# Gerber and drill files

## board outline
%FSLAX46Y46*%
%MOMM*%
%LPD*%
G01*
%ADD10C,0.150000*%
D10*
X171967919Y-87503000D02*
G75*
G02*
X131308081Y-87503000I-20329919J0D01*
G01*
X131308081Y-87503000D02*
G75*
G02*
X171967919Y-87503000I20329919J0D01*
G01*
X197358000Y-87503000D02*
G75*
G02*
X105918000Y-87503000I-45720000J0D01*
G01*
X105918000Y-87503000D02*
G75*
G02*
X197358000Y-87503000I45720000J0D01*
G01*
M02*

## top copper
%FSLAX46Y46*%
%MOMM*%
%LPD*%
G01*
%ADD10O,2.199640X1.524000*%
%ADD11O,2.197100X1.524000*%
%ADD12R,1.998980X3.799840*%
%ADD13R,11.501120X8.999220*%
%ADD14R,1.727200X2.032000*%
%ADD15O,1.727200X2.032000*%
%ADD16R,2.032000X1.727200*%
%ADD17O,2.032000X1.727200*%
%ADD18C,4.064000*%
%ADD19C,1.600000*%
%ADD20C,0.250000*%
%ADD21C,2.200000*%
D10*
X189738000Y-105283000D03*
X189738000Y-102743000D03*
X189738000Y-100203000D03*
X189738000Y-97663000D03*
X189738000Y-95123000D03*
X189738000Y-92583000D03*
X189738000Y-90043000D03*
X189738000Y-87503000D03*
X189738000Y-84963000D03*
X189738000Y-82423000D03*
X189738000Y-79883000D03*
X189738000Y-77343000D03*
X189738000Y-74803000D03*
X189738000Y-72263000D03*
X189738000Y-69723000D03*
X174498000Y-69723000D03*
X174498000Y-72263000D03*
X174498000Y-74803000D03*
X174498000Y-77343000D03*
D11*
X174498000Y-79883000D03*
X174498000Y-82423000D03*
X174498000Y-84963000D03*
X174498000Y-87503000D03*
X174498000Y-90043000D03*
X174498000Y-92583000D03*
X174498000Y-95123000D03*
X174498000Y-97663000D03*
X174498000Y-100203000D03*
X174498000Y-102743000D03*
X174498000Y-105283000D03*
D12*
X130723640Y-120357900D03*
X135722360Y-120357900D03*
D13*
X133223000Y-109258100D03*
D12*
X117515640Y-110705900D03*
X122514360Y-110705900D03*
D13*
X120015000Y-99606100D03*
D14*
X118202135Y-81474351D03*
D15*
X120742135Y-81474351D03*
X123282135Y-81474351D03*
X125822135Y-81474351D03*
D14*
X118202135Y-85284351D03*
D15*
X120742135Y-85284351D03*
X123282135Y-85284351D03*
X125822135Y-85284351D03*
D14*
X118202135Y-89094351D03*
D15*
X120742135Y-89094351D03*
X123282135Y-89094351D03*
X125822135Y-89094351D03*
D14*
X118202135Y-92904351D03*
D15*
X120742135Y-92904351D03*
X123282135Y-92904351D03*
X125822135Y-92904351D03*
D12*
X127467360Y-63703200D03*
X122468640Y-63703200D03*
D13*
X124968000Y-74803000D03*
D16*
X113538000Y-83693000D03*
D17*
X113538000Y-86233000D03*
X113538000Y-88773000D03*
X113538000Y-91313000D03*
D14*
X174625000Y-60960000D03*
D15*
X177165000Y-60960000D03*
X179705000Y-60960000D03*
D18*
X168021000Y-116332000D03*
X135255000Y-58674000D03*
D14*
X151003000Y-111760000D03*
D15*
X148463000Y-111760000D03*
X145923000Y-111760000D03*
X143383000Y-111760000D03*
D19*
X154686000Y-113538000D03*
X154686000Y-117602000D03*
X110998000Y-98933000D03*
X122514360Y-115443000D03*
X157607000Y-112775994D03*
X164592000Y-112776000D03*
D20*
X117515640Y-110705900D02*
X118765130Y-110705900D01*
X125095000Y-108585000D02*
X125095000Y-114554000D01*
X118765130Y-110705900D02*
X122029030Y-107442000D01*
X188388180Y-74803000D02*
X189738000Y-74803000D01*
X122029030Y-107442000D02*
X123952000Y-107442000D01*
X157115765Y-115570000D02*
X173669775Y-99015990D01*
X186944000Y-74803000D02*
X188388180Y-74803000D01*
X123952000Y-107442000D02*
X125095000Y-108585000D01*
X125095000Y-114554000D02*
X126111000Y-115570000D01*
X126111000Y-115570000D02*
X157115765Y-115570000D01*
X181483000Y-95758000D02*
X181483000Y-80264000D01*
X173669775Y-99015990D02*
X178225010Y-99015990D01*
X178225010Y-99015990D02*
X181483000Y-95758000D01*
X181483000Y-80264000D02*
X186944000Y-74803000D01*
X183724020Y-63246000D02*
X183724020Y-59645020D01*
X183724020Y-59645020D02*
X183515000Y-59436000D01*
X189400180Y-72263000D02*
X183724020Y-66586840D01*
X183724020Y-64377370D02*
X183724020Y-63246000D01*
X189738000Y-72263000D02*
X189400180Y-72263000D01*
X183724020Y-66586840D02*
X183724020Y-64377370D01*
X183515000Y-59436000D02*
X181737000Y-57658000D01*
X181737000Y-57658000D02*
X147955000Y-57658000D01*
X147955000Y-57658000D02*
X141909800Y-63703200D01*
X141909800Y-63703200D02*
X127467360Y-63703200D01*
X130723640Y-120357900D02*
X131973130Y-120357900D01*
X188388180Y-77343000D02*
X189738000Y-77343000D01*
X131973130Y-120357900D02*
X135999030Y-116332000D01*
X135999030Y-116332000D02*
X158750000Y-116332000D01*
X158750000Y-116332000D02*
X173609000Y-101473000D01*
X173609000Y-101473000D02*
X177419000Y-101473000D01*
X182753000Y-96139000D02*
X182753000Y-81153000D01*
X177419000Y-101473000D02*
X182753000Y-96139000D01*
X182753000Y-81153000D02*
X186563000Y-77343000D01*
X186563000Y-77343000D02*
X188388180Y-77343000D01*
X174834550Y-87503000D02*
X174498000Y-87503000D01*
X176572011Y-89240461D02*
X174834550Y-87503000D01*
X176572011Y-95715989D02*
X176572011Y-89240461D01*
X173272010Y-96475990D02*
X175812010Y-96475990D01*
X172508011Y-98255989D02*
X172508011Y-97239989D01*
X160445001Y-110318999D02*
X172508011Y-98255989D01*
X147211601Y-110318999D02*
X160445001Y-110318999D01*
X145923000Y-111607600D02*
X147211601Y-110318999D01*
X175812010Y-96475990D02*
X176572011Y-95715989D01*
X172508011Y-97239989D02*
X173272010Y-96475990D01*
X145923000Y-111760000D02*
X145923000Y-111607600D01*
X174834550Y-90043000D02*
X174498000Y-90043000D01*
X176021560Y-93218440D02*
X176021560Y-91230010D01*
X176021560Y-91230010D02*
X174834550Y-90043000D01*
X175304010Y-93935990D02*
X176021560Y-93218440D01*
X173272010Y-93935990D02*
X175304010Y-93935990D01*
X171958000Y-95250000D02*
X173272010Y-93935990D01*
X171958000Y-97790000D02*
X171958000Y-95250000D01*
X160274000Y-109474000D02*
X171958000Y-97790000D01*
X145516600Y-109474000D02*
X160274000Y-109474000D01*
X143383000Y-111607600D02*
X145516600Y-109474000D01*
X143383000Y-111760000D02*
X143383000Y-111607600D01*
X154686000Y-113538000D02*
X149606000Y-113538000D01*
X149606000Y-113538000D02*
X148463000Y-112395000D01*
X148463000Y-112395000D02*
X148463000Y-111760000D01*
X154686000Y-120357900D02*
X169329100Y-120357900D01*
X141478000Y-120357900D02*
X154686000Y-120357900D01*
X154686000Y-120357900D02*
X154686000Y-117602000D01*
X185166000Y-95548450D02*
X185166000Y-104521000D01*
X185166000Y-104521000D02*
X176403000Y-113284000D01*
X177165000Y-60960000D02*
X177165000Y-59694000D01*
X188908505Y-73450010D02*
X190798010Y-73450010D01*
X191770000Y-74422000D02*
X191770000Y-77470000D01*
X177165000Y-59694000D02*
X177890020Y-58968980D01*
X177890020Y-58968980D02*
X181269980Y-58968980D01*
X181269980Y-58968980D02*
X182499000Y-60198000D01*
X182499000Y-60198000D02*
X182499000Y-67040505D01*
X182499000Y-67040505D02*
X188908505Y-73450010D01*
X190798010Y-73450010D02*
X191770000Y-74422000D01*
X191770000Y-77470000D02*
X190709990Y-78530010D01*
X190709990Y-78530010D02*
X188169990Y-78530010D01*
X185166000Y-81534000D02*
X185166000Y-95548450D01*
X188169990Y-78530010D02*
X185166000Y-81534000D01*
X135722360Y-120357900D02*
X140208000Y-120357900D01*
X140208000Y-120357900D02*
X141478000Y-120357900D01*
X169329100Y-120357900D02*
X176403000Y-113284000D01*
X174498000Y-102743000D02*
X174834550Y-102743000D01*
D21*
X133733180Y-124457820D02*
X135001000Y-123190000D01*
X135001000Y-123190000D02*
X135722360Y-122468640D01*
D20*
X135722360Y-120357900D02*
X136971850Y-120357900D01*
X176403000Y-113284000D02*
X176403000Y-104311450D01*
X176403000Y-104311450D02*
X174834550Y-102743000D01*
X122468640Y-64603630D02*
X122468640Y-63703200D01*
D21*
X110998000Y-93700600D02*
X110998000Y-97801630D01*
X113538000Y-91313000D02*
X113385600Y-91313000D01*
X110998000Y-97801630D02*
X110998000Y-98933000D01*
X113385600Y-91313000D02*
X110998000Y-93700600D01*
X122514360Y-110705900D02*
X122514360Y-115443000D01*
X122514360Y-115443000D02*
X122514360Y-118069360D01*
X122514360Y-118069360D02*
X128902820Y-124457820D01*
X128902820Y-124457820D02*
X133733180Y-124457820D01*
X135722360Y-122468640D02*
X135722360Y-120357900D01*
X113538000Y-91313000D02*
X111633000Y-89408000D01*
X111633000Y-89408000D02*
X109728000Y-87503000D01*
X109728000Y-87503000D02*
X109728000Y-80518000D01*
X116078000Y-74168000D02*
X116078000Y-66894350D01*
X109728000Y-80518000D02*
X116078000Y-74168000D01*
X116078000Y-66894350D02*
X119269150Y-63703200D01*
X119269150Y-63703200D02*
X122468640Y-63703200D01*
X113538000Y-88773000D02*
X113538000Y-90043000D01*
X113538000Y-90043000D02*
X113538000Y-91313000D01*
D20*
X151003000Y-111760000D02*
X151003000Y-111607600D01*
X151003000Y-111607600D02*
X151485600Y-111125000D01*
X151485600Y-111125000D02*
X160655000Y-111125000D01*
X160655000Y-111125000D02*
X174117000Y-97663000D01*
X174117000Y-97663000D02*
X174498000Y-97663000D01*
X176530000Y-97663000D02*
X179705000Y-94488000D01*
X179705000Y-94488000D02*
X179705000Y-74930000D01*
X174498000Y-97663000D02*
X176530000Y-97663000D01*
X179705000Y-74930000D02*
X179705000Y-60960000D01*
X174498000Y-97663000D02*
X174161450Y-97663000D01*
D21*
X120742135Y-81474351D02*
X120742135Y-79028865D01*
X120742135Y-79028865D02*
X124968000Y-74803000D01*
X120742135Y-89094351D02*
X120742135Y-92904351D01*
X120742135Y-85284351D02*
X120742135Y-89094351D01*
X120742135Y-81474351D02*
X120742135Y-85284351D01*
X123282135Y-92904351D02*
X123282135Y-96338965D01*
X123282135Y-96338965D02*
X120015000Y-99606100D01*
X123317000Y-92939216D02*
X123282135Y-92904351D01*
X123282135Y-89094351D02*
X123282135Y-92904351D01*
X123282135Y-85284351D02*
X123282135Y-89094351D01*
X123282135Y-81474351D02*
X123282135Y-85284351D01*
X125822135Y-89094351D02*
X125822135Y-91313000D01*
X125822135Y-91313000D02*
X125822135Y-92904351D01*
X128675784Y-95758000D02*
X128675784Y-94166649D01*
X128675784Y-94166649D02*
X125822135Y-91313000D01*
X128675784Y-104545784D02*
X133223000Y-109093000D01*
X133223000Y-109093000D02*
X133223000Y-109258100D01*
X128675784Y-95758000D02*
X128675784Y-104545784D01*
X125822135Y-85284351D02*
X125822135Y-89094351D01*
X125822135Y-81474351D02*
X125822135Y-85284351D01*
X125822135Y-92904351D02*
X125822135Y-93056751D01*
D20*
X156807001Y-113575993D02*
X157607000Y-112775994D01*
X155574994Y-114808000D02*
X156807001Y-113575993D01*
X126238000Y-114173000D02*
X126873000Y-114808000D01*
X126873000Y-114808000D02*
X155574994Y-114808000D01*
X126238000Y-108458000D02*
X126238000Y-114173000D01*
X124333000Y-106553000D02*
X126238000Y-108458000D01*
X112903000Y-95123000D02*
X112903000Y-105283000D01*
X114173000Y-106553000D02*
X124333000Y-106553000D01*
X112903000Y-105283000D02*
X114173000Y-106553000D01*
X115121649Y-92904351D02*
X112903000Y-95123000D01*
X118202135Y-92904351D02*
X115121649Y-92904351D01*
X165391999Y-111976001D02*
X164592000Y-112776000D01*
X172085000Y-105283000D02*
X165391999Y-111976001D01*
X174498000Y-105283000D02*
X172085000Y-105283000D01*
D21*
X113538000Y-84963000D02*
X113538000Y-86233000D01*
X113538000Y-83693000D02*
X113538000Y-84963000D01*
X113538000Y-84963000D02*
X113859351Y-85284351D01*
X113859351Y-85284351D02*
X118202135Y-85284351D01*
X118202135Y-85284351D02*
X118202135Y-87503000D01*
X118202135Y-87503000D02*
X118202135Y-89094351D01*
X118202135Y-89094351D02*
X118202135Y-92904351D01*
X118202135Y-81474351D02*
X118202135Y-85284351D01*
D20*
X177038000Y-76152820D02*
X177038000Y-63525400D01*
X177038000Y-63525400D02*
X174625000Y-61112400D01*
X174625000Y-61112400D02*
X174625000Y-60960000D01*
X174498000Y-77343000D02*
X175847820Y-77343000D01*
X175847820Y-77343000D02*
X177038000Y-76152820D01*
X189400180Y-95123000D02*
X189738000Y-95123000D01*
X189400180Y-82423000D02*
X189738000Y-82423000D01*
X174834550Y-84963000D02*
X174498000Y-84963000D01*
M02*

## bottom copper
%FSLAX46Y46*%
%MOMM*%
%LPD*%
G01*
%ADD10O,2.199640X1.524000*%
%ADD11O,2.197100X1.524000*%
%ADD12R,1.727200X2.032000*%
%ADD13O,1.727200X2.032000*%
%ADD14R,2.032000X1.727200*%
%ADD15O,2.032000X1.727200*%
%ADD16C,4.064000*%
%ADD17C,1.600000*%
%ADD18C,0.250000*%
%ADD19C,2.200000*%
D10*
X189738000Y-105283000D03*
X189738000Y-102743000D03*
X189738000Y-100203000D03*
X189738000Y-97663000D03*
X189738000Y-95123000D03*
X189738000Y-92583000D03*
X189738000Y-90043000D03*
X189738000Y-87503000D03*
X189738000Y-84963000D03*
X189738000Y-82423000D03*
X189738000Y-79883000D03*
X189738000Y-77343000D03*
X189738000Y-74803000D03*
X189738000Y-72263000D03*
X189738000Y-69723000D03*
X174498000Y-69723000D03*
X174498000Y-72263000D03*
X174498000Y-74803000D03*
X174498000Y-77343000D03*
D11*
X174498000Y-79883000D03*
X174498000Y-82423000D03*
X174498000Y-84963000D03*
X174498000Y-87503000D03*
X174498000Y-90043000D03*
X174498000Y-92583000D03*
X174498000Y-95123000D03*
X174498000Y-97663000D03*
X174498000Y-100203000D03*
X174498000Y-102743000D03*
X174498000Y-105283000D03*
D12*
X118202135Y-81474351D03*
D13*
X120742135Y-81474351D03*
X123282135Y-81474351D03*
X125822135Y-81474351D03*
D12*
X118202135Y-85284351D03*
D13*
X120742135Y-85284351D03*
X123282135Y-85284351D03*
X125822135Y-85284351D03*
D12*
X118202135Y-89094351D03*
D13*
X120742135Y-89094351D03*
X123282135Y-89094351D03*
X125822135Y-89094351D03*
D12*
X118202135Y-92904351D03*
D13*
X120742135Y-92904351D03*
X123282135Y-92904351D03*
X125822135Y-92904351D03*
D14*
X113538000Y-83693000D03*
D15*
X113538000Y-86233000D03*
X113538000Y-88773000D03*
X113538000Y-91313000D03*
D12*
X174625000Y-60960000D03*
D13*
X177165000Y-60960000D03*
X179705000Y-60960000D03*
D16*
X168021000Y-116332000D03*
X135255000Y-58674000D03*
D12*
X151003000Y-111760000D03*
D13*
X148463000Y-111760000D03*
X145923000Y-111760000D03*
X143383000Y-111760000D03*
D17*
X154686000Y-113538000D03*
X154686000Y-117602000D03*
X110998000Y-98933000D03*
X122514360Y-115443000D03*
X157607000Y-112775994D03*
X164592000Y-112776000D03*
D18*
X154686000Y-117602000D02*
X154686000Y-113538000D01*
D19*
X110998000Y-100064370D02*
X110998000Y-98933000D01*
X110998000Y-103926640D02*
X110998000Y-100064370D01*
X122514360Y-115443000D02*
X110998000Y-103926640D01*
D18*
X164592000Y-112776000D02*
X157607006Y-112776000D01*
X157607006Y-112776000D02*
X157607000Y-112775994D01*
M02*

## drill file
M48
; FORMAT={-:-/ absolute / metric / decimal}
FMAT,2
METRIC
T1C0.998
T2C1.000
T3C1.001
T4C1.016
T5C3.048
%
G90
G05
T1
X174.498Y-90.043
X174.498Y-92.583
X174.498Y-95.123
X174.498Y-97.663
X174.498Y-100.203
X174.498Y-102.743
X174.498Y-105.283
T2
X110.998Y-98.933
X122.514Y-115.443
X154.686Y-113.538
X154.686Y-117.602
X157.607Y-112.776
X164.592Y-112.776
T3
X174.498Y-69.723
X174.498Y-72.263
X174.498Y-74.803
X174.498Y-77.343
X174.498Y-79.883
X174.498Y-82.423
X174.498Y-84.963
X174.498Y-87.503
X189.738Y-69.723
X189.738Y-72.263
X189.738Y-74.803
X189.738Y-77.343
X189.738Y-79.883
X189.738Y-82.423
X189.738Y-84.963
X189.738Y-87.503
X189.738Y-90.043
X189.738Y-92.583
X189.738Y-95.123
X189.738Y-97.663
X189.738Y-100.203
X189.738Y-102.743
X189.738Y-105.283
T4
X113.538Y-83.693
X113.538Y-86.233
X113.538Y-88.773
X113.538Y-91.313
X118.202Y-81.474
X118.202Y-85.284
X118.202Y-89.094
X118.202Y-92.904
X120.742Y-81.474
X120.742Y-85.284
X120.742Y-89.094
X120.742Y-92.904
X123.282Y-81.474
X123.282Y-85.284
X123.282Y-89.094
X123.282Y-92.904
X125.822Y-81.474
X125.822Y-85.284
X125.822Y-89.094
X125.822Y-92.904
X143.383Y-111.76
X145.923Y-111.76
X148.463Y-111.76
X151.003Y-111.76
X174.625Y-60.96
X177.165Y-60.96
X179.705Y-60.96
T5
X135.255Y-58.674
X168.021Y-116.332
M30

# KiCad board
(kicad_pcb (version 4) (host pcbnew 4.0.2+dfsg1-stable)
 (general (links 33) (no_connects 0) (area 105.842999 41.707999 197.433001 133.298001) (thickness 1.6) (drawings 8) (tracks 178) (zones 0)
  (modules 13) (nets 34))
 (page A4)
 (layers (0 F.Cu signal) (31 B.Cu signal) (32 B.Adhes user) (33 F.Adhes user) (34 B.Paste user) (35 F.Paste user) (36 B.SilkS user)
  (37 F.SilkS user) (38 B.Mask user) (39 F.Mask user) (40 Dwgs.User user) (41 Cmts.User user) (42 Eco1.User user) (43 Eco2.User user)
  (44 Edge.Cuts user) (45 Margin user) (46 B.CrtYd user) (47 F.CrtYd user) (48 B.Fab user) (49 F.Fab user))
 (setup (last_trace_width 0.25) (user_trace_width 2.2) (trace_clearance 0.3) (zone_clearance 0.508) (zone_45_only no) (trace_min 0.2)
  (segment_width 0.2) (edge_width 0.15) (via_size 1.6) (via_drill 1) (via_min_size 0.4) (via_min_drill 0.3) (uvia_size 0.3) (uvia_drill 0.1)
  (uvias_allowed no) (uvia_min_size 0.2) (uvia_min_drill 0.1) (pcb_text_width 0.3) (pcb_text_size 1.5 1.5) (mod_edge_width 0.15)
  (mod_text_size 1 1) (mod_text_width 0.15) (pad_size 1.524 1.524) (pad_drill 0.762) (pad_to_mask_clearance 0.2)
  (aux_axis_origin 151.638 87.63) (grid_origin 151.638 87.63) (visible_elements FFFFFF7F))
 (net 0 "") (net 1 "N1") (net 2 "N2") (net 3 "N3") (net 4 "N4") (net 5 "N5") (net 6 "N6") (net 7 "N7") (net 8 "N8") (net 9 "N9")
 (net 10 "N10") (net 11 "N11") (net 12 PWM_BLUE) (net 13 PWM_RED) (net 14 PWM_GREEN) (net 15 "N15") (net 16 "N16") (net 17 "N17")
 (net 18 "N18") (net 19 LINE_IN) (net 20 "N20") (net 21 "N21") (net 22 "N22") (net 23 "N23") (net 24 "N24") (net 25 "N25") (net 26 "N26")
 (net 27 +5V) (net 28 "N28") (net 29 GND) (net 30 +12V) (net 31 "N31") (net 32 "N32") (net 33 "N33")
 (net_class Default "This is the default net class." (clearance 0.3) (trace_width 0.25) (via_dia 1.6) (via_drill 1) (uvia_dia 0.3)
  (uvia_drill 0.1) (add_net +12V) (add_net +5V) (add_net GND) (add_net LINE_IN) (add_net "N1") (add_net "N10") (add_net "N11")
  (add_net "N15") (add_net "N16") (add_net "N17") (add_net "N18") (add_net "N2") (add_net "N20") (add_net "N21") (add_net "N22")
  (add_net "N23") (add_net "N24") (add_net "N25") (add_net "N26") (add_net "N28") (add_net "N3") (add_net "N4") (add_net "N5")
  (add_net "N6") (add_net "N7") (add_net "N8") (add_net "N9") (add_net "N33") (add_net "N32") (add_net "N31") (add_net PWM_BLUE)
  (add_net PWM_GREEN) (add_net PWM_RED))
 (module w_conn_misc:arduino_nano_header (layer F.Cu) (at 182.118 87.503 90)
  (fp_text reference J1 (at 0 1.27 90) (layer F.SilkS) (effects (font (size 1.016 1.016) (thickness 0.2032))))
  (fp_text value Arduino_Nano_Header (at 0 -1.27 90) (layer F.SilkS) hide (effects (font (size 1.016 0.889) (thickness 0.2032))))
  (pad 1 thru_hole oval (at -17.78 7.62 90) (size 1.524 2.19964) (drill 1.00076) (layers *.Cu *.Mask F.SilkS) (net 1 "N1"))
  (pad 2 thru_hole oval (at -15.24 7.62 90) (size 1.524 2.19964) (drill 1.00076) (layers *.Cu *.Mask F.SilkS) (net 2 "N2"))
  (pad 3 thru_hole oval (at -12.7 7.62 90) (size 1.524 2.19964) (drill 1.00076) (layers *.Cu *.Mask F.SilkS) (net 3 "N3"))
  (pad 4 thru_hole oval (at -10.16 7.62 90) (size 1.524 2.19964) (drill 1.00076) (layers *.Cu *.Mask F.SilkS) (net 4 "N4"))
  (pad 5 thru_hole oval (at -7.62 7.62 90) (size 1.524 2.19964) (drill 1.00076) (layers *.Cu *.Mask F.SilkS) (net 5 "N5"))
  (pad 6 thru_hole oval (at -5.08 7.62 90) (size 1.524 2.19964) (drill 1.00076) (layers *.Cu *.Mask F.SilkS) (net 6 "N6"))
  (pad 7 thru_hole oval (at -2.54 7.62 90) (size 1.524 2.19964) (drill 1.00076) (layers *.Cu *.Mask F.SilkS) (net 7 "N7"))
  (pad 8 thru_hole oval (at 0 7.62 90) (size 1.524 2.19964) (drill 1.00076) (layers *.Cu *.Mask F.SilkS) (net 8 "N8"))
  (pad 9 thru_hole oval (at 2.54 7.62 90) (size 1.524 2.19964) (drill 1.00076) (layers *.Cu *.Mask F.SilkS) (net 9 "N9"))
  (pad 10 thru_hole oval (at 5.08 7.62 90) (size 1.524 2.19964) (drill 1.00076) (layers *.Cu *.Mask F.SilkS) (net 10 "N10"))
  (pad 11 thru_hole oval (at 7.62 7.62 90) (size 1.524 2.19964) (drill 1.00076) (layers *.Cu *.Mask F.SilkS) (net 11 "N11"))
  (pad 12 thru_hole oval (at 10.16 7.62 90) (size 1.524 2.19964) (drill 1.00076) (layers *.Cu *.Mask F.SilkS) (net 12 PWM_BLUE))
  (pad 13 thru_hole oval (at 12.7 7.62 90) (size 1.524 2.19964) (drill 1.00076) (layers *.Cu *.Mask F.SilkS) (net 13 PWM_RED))
  (pad 14 thru_hole oval (at 15.24 7.62 90) (size 1.524 2.19964) (drill 1.00076) (layers *.Cu *.Mask F.SilkS) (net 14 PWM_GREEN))
  (pad 15 thru_hole oval (at 17.78 7.62 90) (size 1.524 2.19964) (drill 1.00076) (layers *.Cu *.Mask F.SilkS) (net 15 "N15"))
  (pad 16 thru_hole oval (at 17.78 -7.62 90) (size 1.524 2.19964) (drill 1.00076) (layers *.Cu *.Mask F.SilkS) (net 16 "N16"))
  (pad 17 thru_hole oval (at 15.24 -7.62 90) (size 1.524 2.19964) (drill 1.00076) (layers *.Cu *.Mask F.SilkS) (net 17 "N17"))
  (pad 18 thru_hole oval (at 12.7 -7.62 90) (size 1.524 2.19964) (drill 1.00076) (layers *.Cu *.Mask F.SilkS) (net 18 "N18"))
  (pad 19 thru_hole oval (at 10.16 -7.62 90) (size 1.524 2.19964) (drill 1.00076) (layers *.Cu *.Mask F.SilkS) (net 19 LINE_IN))
  (pad 20 thru_hole oval (at 7.62 -7.62 90) (size 1.524 2.1971) (drill 1.00076) (layers *.Cu *.Mask F.SilkS) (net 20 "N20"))
  (pad 21 thru_hole oval (at 5.08 -7.62 90) (size 1.524 2.1971) (drill 1.00076) (layers *.Cu *.Mask F.SilkS) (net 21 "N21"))
  (pad 22 thru_hole oval (at 2.54 -7.62 90) (size 1.524 2.1971) (drill 1.00076) (layers *.Cu *.Mask F.SilkS) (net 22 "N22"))
  (pad 23 thru_hole oval (at 0 -7.62 90) (size 1.524 2.1971) (drill 1.00076) (layers *.Cu *.Mask F.SilkS) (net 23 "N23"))
  (pad 24 thru_hole oval (at -2.54 -7.62 90) (size 1.524 2.1971) (drill 0.99822) (layers *.Cu *.Mask F.SilkS) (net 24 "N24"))
  (pad 25 thru_hole oval (at -5.08 -7.62 90) (size 1.524 2.1971) (drill 0.99822) (layers *.Cu *.Mask F.SilkS) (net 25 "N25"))
  (pad 26 thru_hole oval (at -7.62 -7.62 90) (size 1.524 2.1971) (drill 0.99822) (layers *.Cu *.Mask F.SilkS) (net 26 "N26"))
  (pad 27 thru_hole oval (at -10.16 -7.62 90) (size 1.524 2.1971) (drill 0.99822) (layers *.Cu *.Mask F.SilkS) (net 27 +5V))
  (pad 28 thru_hole oval (at -12.7 -7.62 90) (size 1.524 2.1971) (drill 0.99822) (layers *.Cu *.Mask F.SilkS) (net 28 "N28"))
  (pad 29 thru_hole oval (at -15.24 -7.62 90) (size 1.524 2.1971) (drill 0.99822) (layers *.Cu *.Mask F.SilkS) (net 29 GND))
  (pad 30 thru_hole oval (at -17.78 -7.62 90) (size 1.524 2.1971) (drill 0.99822) (layers *.Cu *.Mask F.SilkS) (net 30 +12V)))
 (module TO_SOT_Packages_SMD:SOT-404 (layer F.Cu) (at 133.223 114.808)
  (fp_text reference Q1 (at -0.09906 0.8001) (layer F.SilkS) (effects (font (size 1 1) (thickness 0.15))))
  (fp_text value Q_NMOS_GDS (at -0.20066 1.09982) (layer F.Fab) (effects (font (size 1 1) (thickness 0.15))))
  (pad 1 smd rect (at -2.49936 5.5499) (size 1.99898 3.79984) (layers F.Cu F.Paste F.Mask) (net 12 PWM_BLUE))
  (pad 3 smd rect (at 2.49936 5.5499) (size 1.99898 3.79984) (layers F.Cu F.Paste F.Mask) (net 29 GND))
  (pad 2 smd rect (at 0 -5.5499) (size 11.50112 8.99922) (layers F.Cu F.Paste F.Mask) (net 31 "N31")))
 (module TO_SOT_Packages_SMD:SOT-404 (layer F.Cu) (at 120.015 105.156)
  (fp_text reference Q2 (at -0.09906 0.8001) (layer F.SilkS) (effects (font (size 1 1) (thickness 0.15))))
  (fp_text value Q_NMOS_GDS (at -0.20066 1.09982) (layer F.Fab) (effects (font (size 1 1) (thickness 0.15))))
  (pad 1 smd rect (at -2.49936 5.5499) (size 1.99898 3.79984) (layers F.Cu F.Paste F.Mask) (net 13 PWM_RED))
  (pad 3 smd rect (at 2.49936 5.5499) (size 1.99898 3.79984) (layers F.Cu F.Paste F.Mask) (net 29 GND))
  (pad 2 smd rect (at 0 -5.5499) (size 11.50112 8.99922) (layers F.Cu F.Paste F.Mask) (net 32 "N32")))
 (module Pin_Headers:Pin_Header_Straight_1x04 (layer F.Cu) (at 118.202135 81.474351 90)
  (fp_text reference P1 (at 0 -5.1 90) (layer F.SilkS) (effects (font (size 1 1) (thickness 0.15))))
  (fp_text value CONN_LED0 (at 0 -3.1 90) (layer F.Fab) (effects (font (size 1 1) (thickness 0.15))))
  (pad 1 thru_hole rect (at 0 0 90) (size 2.032 1.7272) (drill 1.016) (layers *.Cu *.Mask F.SilkS) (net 30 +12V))
  (pad 2 thru_hole oval (at 0 2.54 90) (size 2.032 1.7272) (drill 1.016) (layers *.Cu *.Mask F.SilkS) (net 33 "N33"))
  (pad 3 thru_hole oval (at 0 5.08 90) (size 2.032 1.7272) (drill 1.016) (layers *.Cu *.Mask F.SilkS) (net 32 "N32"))
  (pad 4 thru_hole oval (at 0 7.62 90) (size 2.032 1.7272) (drill 1.016) (layers *.Cu *.Mask F.SilkS) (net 31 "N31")))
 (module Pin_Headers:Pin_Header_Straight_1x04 (layer F.Cu) (at 118.202135 85.284351 90)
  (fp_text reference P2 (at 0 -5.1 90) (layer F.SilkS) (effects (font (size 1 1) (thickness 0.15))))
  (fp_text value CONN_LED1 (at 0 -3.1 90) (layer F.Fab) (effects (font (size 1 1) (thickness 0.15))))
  (pad 1 thru_hole rect (at 0 0 90) (size 2.032 1.7272) (drill 1.016) (layers *.Cu *.Mask F.SilkS) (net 30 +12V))
  (pad 2 thru_hole oval (at 0 2.54 90) (size 2.032 1.7272) (drill 1.016) (layers *.Cu *.Mask F.SilkS) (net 33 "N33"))
  (pad 3 thru_hole oval (at 0 5.08 90) (size 2.032 1.7272) (drill 1.016) (layers *.Cu *.Mask F.SilkS) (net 32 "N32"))
  (pad 4 thru_hole oval (at 0 7.62 90) (size 2.032 1.7272) (drill 1.016) (layers *.Cu *.Mask F.SilkS) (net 31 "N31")))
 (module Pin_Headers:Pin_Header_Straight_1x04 (layer F.Cu) (at 118.202135 89.094351 90)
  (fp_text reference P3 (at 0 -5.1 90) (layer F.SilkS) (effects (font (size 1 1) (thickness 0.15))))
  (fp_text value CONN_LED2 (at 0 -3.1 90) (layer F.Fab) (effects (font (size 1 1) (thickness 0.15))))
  (pad 1 thru_hole rect (at 0 0 90) (size 2.032 1.7272) (drill 1.016) (layers *.Cu *.Mask F.SilkS) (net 30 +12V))
  (pad 2 thru_hole oval (at 0 2.54 90) (size 2.032 1.7272) (drill 1.016) (layers *.Cu *.Mask F.SilkS) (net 33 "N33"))
  (pad 3 thru_hole oval (at 0 5.08 90) (size 2.032 1.7272) (drill 1.016) (layers *.Cu *.Mask F.SilkS) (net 32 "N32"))
  (pad 4 thru_hole oval (at 0 7.62 90) (size 2.032 1.7272) (drill 1.016) (layers *.Cu *.Mask F.SilkS) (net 31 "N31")))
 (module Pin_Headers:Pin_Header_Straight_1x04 (layer F.Cu) (at 118.202135 92.904351 90)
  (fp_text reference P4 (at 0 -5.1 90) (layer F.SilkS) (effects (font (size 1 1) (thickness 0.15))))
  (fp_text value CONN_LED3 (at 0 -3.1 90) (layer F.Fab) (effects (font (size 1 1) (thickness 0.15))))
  (pad 1 thru_hole rect (at 0 0 90) (size 2.032 1.7272) (drill 1.016) (layers *.Cu *.Mask F.SilkS) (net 30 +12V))
  (pad 2 thru_hole oval (at 0 2.54 90) (size 2.032 1.7272) (drill 1.016) (layers *.Cu *.Mask F.SilkS) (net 33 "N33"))
  (pad 3 thru_hole oval (at 0 5.08 90) (size 2.032 1.7272) (drill 1.016) (layers *.Cu *.Mask F.SilkS) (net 32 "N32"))
  (pad 4 thru_hole oval (at 0 7.62 90) (size 2.032 1.7272) (drill 1.016) (layers *.Cu *.Mask F.SilkS) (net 31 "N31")))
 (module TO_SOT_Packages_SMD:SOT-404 (layer F.Cu) (at 124.968 69.2531 180)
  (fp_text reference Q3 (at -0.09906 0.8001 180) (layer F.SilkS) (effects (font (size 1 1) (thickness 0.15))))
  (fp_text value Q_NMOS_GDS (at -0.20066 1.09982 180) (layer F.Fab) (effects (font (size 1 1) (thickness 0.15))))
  (pad 1 smd rect (at -2.49936 5.5499 180) (size 1.99898 3.79984) (layers F.Cu F.Paste F.Mask) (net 14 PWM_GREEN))
  (pad 3 smd rect (at 2.49936 5.5499 180) (size 1.99898 3.79984) (layers F.Cu F.Paste F.Mask) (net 29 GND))
  (pad 2 smd rect (at 0 -5.5499 180) (size 11.50112 8.99922) (layers F.Cu F.Paste F.Mask) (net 33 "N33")))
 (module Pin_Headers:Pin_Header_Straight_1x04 (layer F.Cu) (at 113.538 83.693)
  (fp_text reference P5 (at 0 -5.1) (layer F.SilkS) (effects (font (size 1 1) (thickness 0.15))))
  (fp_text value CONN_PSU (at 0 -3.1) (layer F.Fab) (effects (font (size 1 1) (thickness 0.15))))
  (pad 1 thru_hole rect (at 0 0) (size 2.032 1.7272) (drill 1.016) (layers *.Cu *.Mask F.SilkS) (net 30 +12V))
  (pad 2 thru_hole oval (at 0 2.54) (size 2.032 1.7272) (drill 1.016) (layers *.Cu *.Mask F.SilkS) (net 30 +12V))
  (pad 3 thru_hole oval (at 0 5.08) (size 2.032 1.7272) (drill 1.016) (layers *.Cu *.Mask F.SilkS) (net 29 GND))
  (pad 4 thru_hole oval (at 0 7.62) (size 2.032 1.7272) (drill 1.016) (layers *.Cu *.Mask F.SilkS) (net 29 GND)))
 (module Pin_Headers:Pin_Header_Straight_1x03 (layer F.Cu) (at 174.625 60.96 90)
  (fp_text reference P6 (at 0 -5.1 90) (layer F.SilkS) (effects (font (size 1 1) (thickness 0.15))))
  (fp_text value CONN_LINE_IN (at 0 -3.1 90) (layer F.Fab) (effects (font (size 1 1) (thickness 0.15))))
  (pad 1 thru_hole rect (at 0 0 90) (size 2.032 1.7272) (drill 1.016) (layers *.Cu *.Mask F.SilkS) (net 19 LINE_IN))
  (pad 2 thru_hole oval (at 0 2.54 90) (size 2.032 1.7272) (drill 1.016) (layers *.Cu *.Mask F.SilkS) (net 29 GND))
  (pad 3 thru_hole oval (at 0 5.08 90) (size 2.032 1.7272) (drill 1.016) (layers *.Cu *.Mask F.SilkS) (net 27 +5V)))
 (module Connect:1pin (layer F.Cu) (at 168.021 116.332)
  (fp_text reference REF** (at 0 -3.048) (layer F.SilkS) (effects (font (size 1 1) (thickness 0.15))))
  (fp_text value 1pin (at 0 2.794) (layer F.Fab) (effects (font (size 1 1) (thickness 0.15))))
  (pad 1 thru_hole circle (at 0 0) (size 4.064 4.064) (drill 3.048) (layers *.Cu *.Mask F.SilkS)))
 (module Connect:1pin (layer F.Cu) (at 135.255 58.674)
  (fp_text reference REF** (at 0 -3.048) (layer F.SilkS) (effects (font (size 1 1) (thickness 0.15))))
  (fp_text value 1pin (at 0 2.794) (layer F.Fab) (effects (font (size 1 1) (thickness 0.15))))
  (pad 1 thru_hole circle (at 0 0) (size 4.064 4.064) (drill 3.048) (layers *.Cu *.Mask F.SilkS)))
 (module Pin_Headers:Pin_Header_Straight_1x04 (layer F.Cu) (at 151.003 111.76 270)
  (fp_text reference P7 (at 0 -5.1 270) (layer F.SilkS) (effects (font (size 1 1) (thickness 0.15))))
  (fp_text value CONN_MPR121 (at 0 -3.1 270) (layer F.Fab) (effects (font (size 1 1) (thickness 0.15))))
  (pad 1 thru_hole rect (at 0 0 270) (size 2.032 1.7272) (drill 1.016) (layers *.Cu *.Mask F.SilkS) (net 27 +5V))
  (pad 2 thru_hole oval (at 0 2.54 270) (size 2.032 1.7272) (drill 1.016) (layers *.Cu *.Mask F.SilkS) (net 29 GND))
  (pad 3 thru_hole oval (at 0 5.08 270) (size 2.032 1.7272) (drill 1.016) (layers *.Cu *.Mask F.SilkS) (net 23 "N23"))
  (pad 4 thru_hole oval (at 0 7.62 270) (size 2.032 1.7272) (drill 1.016) (layers *.Cu *.Mask F.SilkS) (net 24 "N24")))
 (gr_circle (center 151.638 87.503) (end 171.958 88.138) (layer Edge.Cuts) (width 0.15))
 (gr_circle (center 151.638 87.503) (end 197.358 87.503) (layer Edge.Cuts) (width 0.15))
 (segment (start 117.51564 110.7059) (end 118.76513 110.7059) (width 0.25) (layer F.Cu) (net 13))
 (segment (start 125.095 108.585) (end 125.095 114.554) (width 0.25) (layer F.Cu) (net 13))
 (segment (start 118.76513 110.7059) (end 122.02903 107.442) (width 0.25) (layer F.Cu) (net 13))
 (segment (start 188.38818 74.803) (end 189.738 74.803) (width 0.25) (layer F.Cu) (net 13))
 (segment (start 122.02903 107.442) (end 123.952 107.442) (width 0.25) (layer F.Cu) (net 13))
 (segment (start 157.115765 115.57) (end 173.669775 99.01599) (width 0.25) (layer F.Cu) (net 13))
 (segment (start 186.944 74.803) (end 188.38818 74.803) (width 0.25) (layer F.Cu) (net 13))
 (segment (start 123.952 107.442) (end 125.095 108.585) (width 0.25) (layer F.Cu) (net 13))
 (segment (start 125.095 114.554) (end 126.111 115.57) (width 0.25) (layer F.Cu) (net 13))
 (segment (start 126.111 115.57) (end 157.115765 115.57) (width 0.25) (layer F.Cu) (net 13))
 (segment (start 181.483 95.758) (end 181.483 80.264) (width 0.25) (layer F.Cu) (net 13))
 (segment (start 173.669775 99.01599) (end 178.22501 99.01599) (width 0.25) (layer F.Cu) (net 13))
 (segment (start 178.22501 99.01599) (end 181.483 95.758) (width 0.25) (layer F.Cu) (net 13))
 (segment (start 181.483 80.264) (end 186.944 74.803) (width 0.25) (layer F.Cu) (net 13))
 (segment (start 183.72402 63.246) (end 183.72402 59.64502) (width 0.25) (layer F.Cu) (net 14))
 (segment (start 183.72402 59.64502) (end 183.515 59.436) (width 0.25) (layer F.Cu) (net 14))
 (segment (start 189.40018 72.263) (end 183.72402 66.58684) (width 0.25) (layer F.Cu) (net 14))
 (segment (start 183.72402 64.37737) (end 183.72402 63.246) (width 0.25) (layer F.Cu) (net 14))
 (segment (start 189.738 72.263) (end 189.40018 72.263) (width 0.25) (layer F.Cu) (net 14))
 (segment (start 183.72402 66.58684) (end 183.72402 64.37737) (width 0.25) (layer F.Cu) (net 14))
 (segment (start 183.515 59.436) (end 181.737 57.658) (width 0.25) (layer F.Cu) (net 14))
 (segment (start 181.737 57.658) (end 147.955 57.658) (width 0.25) (layer F.Cu) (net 14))
 (segment (start 147.955 57.658) (end 141.9098 63.7032) (width 0.25) (layer F.Cu) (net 14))
 (segment (start 141.9098 63.7032) (end 127.46736 63.7032) (width 0.25) (layer F.Cu) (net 14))
 (segment (start 130.72364 120.3579) (end 131.97313 120.3579) (width 0.25) (layer F.Cu) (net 12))
 (segment (start 188.38818 77.343) (end 189.738 77.343) (width 0.25) (layer F.Cu) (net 12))
 (segment (start 131.97313 120.3579) (end 135.99903 116.332) (width 0.25) (layer F.Cu) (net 12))
 (segment (start 135.99903 116.332) (end 158.75 116.332) (width 0.25) (layer F.Cu) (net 12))
 (segment (start 158.75 116.332) (end 173.609 101.473) (width 0.25) (layer F.Cu) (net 12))
 (segment (start 173.609 101.473) (end 177.419 101.473) (width 0.25) (layer F.Cu) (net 12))
 (segment (start 182.753 96.139) (end 182.753 81.153) (width 0.25) (layer F.Cu) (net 12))
 (segment (start 177.419 101.473) (end 182.753 96.139) (width 0.25) (layer F.Cu) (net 12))
 (segment (start 182.753 81.153) (end 186.563 77.343) (width 0.25) (layer F.Cu) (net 12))
 (segment (start 186.563 77.343) (end 188.38818 77.343) (width 0.25) (layer F.Cu) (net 12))
 (segment (start 174.83455 87.503) (end 174.498 87.503) (width 0.25) (layer F.Cu) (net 23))
 (segment (start 176.572011 89.240461) (end 174.83455 87.503) (width 0.25) (layer F.Cu) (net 23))
 (segment (start 176.572011 95.715989) (end 176.572011 89.240461) (width 0.25) (layer F.Cu) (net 23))
 (segment (start 173.27201 96.47599) (end 175.81201 96.47599) (width 0.25) (layer F.Cu) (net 23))
 (segment (start 172.508011 98.255989) (end 172.508011 97.239989) (width 0.25) (layer F.Cu) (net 23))
 (segment (start 160.445001 110.318999) (end 172.508011 98.255989) (width 0.25) (layer F.Cu) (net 23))
 (segment (start 147.211601 110.318999) (end 160.445001 110.318999) (width 0.25) (layer F.Cu) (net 23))
 (segment (start 145.923 111.6076) (end 147.211601 110.318999) (width 0.25) (layer F.Cu) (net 23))
 (segment (start 175.81201 96.47599) (end 176.572011 95.715989) (width 0.25) (layer F.Cu) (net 23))
 (segment (start 172.508011 97.239989) (end 173.27201 96.47599) (width 0.25) (layer F.Cu) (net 23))
 (segment (start 145.923 111.76) (end 145.923 111.6076) (width 0.25) (layer F.Cu) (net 23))
 (segment (start 174.83455 90.043) (end 174.498 90.043) (width 0.25) (layer F.Cu) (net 24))
 (segment (start 176.02156 93.21844) (end 176.02156 91.23001) (width 0.25) (layer F.Cu) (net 24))
 (segment (start 176.02156 91.23001) (end 174.83455 90.043) (width 0.25) (layer F.Cu) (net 24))
 (segment (start 175.30401 93.93599) (end 176.02156 93.21844) (width 0.25) (layer F.Cu) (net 24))
 (segment (start 173.27201 93.93599) (end 175.30401 93.93599) (width 0.25) (layer F.Cu) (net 24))
 (segment (start 171.958 95.25) (end 173.27201 93.93599) (width 0.25) (layer F.Cu) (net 24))
 (segment (start 171.958 97.79) (end 171.958 95.25) (width 0.25) (layer F.Cu) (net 24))
 (segment (start 160.274 109.474) (end 171.958 97.79) (width 0.25) (layer F.Cu) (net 24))
 (segment (start 145.5166 109.474) (end 160.274 109.474) (width 0.25) (layer F.Cu) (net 24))
 (segment (start 143.383 111.6076) (end 145.5166 109.474) (width 0.25) (layer F.Cu) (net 24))
 (segment (start 143.383 111.76) (end 143.383 111.6076) (width 0.25) (layer F.Cu) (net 24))
 (segment (start 154.686 113.538) (end 149.606 113.538) (width 0.25) (layer F.Cu) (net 29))
 (segment (start 149.606 113.538) (end 148.463 112.395) (width 0.25) (layer F.Cu) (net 29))
 (segment (start 148.463 112.395) (end 148.463 111.76) (width 0.25) (layer F.Cu) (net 29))
 (segment (start 154.686 117.602) (end 154.686 113.538) (width 0.25) (layer B.Cu) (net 29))
 (via (at 154.686 113.538) (size 1.6) (drill 1) (layers F.Cu B.Cu) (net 29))
 (segment (start 154.686 120.3579) (end 169.3291 120.3579) (width 0.25) (layer F.Cu) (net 29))
 (segment (start 141.478 120.3579) (end 154.686 120.3579) (width 0.25) (layer F.Cu) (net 29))
 (segment (start 154.686 120.3579) (end 154.686 117.602) (width 0.25) (layer F.Cu) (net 29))
 (via (at 154.686 117.602) (size 1.6) (drill 1) (layers F.Cu B.Cu) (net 29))
 (segment (start 185.166 95.54845) (end 185.166 104.521) (width 0.25) (layer F.Cu) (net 29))
 (segment (start 185.166 104.521) (end 176.403 113.284) (width 0.25) (layer F.Cu) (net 29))
 (segment (start 177.165 60.96) (end 177.165 59.694) (width 0.25) (layer F.Cu) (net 29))
 (segment (start 188.908505 73.45001) (end 190.79801 73.45001) (width 0.25) (layer F.Cu) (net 29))
 (segment (start 191.77 74.422) (end 191.77 77.47) (width 0.25) (layer F.Cu) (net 29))
 (segment (start 177.165 59.694) (end 177.89002 58.96898) (width 0.25) (layer F.Cu) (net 29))
 (segment (start 177.89002 58.96898) (end 181.26998 58.96898) (width 0.25) (layer F.Cu) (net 29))
 (segment (start 181.26998 58.96898) (end 182.499 60.198) (width 0.25) (layer F.Cu) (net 29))
 (segment (start 182.499 60.198) (end 182.499 67.040505) (width 0.25) (layer F.Cu) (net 29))
 (segment (start 182.499 67.040505) (end 188.908505 73.45001) (width 0.25) (layer F.Cu) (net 29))
 (segment (start 190.79801 73.45001) (end 191.77 74.422) (width 0.25) (layer F.Cu) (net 29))
 (segment (start 191.77 77.47) (end 190.70999 78.53001) (width 0.25) (layer F.Cu) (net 29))
 (segment (start 190.70999 78.53001) (end 188.16999 78.53001) (width 0.25) (layer F.Cu) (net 29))
 (segment (start 185.166 81.534) (end 185.166 95.54845) (width 0.25) (layer F.Cu) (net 29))
 (segment (start 188.16999 78.53001) (end 185.166 81.534) (width 0.25) (layer F.Cu) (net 29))
 (segment (start 135.72236 120.3579) (end 140.208 120.3579) (width 0.25) (layer F.Cu) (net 29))
 (segment (start 140.208 120.3579) (end 141.478 120.3579) (width 0.25) (layer F.Cu) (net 29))
 (segment (start 169.3291 120.3579) (end 176.403 113.284) (width 0.25) (layer F.Cu) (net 29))
 (segment (start 174.498 102.743) (end 174.83455 102.743) (width 0.25) (layer F.Cu) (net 29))
 (segment (start 133.73318 124.45782) (end 135.001 123.19) (width 2.2) (layer F.Cu) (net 29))
 (segment (start 135.001 123.19) (end 135.72236 122.46864) (width 2.2) (layer F.Cu) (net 29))
 (segment (start 135.72236 120.3579) (end 136.97185 120.3579) (width 0.25) (layer F.Cu) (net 29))
 (segment (start 176.403 113.284) (end 176.403 104.31145) (width 0.25) (layer F.Cu) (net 29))
 (segment (start 176.403 104.31145) (end 174.83455 102.743) (width 0.25) (layer F.Cu) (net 29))
 (segment (start 122.46864 64.60363) (end 122.46864 63.7032) (width 0.25) (layer F.Cu) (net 29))
 (segment (start 110.998 100.06437) (end 110.998 98.933) (width 2.2) (layer B.Cu) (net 29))
 (segment (start 110.998 103.92664) (end 110.998 100.06437) (width 2.2) (layer B.Cu) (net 29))
 (segment (start 122.51436 115.443) (end 110.998 103.92664) (width 2.2) (layer B.Cu) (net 29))
 (segment (start 110.998 93.7006) (end 110.998 97.80163) (width 2.2) (layer F.Cu) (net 29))
 (segment (start 113.538 91.313) (end 113.3856 91.313) (width 2.2) (layer F.Cu) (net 29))
 (segment (start 110.998 97.80163) (end 110.998 98.933) (width 2.2) (layer F.Cu) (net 29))
 (segment (start 113.3856 91.313) (end 110.998 93.7006) (width 2.2) (layer F.Cu) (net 29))
 (via (at 110.998 98.933) (size 1.6) (drill 1) (layers F.Cu B.Cu) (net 29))
 (segment (start 122.51436 110.7059) (end 122.51436 115.443) (width 2.2) (layer F.Cu) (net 29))
 (segment (start 122.51436 115.443) (end 122.51436 118.06936) (width 2.2) (layer F.Cu) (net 29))
 (via (at 122.51436 115.443) (size 1.6) (drill 1) (layers F.Cu B.Cu) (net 29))
 (segment (start 122.51436 118.06936) (end 128.90282 124.45782) (width 2.2) (layer F.Cu) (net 29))
 (segment (start 128.90282 124.45782) (end 133.73318 124.45782) (width 2.2) (layer F.Cu) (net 29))
 (segment (start 135.72236 122.46864) (end 135.72236 120.3579) (width 2.2) (layer F.Cu) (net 29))
 (segment (start 113.538 91.313) (end 111.633 89.408) (width 2.2) (layer F.Cu) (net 29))
 (segment (start 111.633 89.408) (end 109.728 87.503) (width 2.2) (layer F.Cu) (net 29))
 (segment (start 109.728 87.503) (end 109.728 80.518) (width 2.2) (layer F.Cu) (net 29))
 (segment (start 116.078 74.168) (end 116.078 66.89435) (width 2.2) (layer F.Cu) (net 29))
 (segment (start 109.728 80.518) (end 116.078 74.168) (width 2.2) (layer F.Cu) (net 29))
 (segment (start 116.078 66.89435) (end 119.26915 63.7032) (width 2.2) (layer F.Cu) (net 29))
 (segment (start 119.26915 63.7032) (end 122.46864 63.7032) (width 2.2) (layer F.Cu) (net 29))
 (segment (start 113.538 88.773) (end 113.538 90.043) (width 2.2) (layer F.Cu) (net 29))
 (segment (start 113.538 90.043) (end 113.538 91.313) (width 2.2) (layer F.Cu) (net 29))
 (segment (start 151.003 111.76) (end 151.003 111.6076) (width 0.25) (layer F.Cu) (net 27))
 (segment (start 151.003 111.6076) (end 151.4856 111.125) (width 0.25) (layer F.Cu) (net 27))
 (segment (start 151.4856 111.125) (end 160.655 111.125) (width 0.25) (layer F.Cu) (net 27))
 (segment (start 160.655 111.125) (end 174.117 97.663) (width 0.25) (layer F.Cu) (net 27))
 (segment (start 174.117 97.663) (end 174.498 97.663) (width 0.25) (layer F.Cu) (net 27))
 (segment (start 176.53 97.663) (end 179.705 94.488) (width 0.25) (layer F.Cu) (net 27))
 (segment (start 179.705 94.488) (end 179.705 74.93) (width 0.25) (layer F.Cu) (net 27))
 (segment (start 174.498 97.663) (end 176.53 97.663) (width 0.25) (layer F.Cu) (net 27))
 (segment (start 179.705 74.93) (end 179.705 60.96) (width 0.25) (layer F.Cu) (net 27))
 (segment (start 174.498 97.663) (end 174.16145 97.663) (width 0.25) (layer F.Cu) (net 27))
 (segment (start 120.742135 81.474351) (end 120.742135 79.028865) (width 2.2) (layer F.Cu) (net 33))
 (segment (start 120.742135 79.028865) (end 124.968 74.803) (width 2.2) (layer F.Cu) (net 33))
 (segment (start 120.742135 89.094351) (end 120.742135 92.904351) (width 2.2) (layer F.Cu) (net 33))
 (segment (start 120.742135 85.284351) (end 120.742135 89.094351) (width 2.2) (layer F.Cu) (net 33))
 (segment (start 120.742135 81.474351) (end 120.742135 85.284351) (width 2.2) (layer F.Cu) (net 33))
 (segment (start 123.282135 92.904351) (end 123.282135 96.338965) (width 2.2) (layer F.Cu) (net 32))
 (segment (start 123.282135 96.338965) (end 120.015 99.6061) (width 2.2) (layer F.Cu) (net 32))
 (segment (start 123.317 92.939216) (end 123.282135 92.904351) (width 2.2) (layer F.Cu) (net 32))
 (segment (start 123.282135 89.094351) (end 123.282135 92.904351) (width 2.2) (layer F.Cu) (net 32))
 (segment (start 123.282135 85.284351) (end 123.282135 89.094351) (width 2.2) (layer F.Cu) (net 32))
 (segment (start 123.282135 81.474351) (end 123.282135 85.284351) (width 2.2) (layer F.Cu) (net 32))
 (segment (start 125.822135 89.094351) (end 125.822135 91.313) (width 2.2) (layer F.Cu) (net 31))
 (segment (start 125.822135 91.313) (end 125.822135 92.904351) (width 2.2) (layer F.Cu) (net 31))
 (segment (start 128.675784 95.758) (end 128.675784 94.166649) (width 2.2) (layer F.Cu) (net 31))
 (segment (start 128.675784 94.166649) (end 125.822135 91.313) (width 2.2) (layer F.Cu) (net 31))
 (segment (start 128.675784 104.545784) (end 133.223 109.093) (width 2.2) (layer F.Cu) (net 31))
 (segment (start 133.223 109.093) (end 133.223 109.2581) (width 2.2) (layer F.Cu) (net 31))
 (segment (start 128.675784 95.758) (end 128.675784 104.545784) (width 2.2) (layer F.Cu) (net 31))
 (segment (start 125.822135 85.284351) (end 125.822135 89.094351) (width 2.2) (layer F.Cu) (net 31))
 (segment (start 125.822135 81.474351) (end 125.822135 85.284351) (width 2.2) (layer F.Cu) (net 31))
 (segment (start 125.822135 92.904351) (end 125.822135 93.056751) (width 2.2) (layer F.Cu) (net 31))
 (segment (start 156.807001 113.575993) (end 157.607 112.775994) (width 0.25) (layer F.Cu) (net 30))
 (segment (start 155.574994 114.808) (end 156.807001 113.575993) (width 0.25) (layer F.Cu) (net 30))
 (segment (start 126.238 114.173) (end 126.873 114.808) (width 0.25) (layer F.Cu) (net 30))
 (segment (start 126.873 114.808) (end 155.574994 114.808) (width 0.25) (layer F.Cu) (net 30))
 (segment (start 126.238 108.458) (end 126.238 114.173) (width 0.25) (layer F.Cu) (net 30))
 (segment (start 124.333 106.553) (end 126.238 108.458) (width 0.25) (layer F.Cu) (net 30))
 (segment (start 112.903 95.123) (end 112.903 105.283) (width 0.25) (layer F.Cu) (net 30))
 (segment (start 114.173 106.553) (end 124.333 106.553) (width 0.25) (layer F.Cu) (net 30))
 (segment (start 112.903 105.283) (end 114.173 106.553) (width 0.25) (layer F.Cu) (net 30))
 (segment (start 115.121649 92.904351) (end 112.903 95.123) (width 0.25) (layer F.Cu) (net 30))
 (segment (start 118.202135 92.904351) (end 115.121649 92.904351) (width 0.25) (layer F.Cu) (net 30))
 (segment (start 164.592 112.776) (end 157.607006 112.776) (width 0.25) (layer B.Cu) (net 30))
 (segment (start 157.607006 112.776) (end 157.607 112.775994) (width 0.25) (layer B.Cu) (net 30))
 (via (at 157.607 112.775994) (size 1.6) (drill 1) (layers F.Cu B.Cu) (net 30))
 (segment (start 165.391999 111.976001) (end 164.592 112.776) (width 0.25) (layer F.Cu) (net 30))
 (segment (start 172.085 105.283) (end 165.391999 111.976001) (width 0.25) (layer F.Cu) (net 30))
 (segment (start 174.498 105.283) (end 172.085 105.283) (width 0.25) (layer F.Cu) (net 30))
 (via (at 164.592 112.776) (size 1.6) (drill 1) (layers F.Cu B.Cu) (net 30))
 (segment (start 113.538 84.963) (end 113.538 86.233) (width 2.2) (layer F.Cu) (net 30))
 (segment (start 113.538 83.693) (end 113.538 84.963) (width 2.2) (layer F.Cu) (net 30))
 (segment (start 113.538 84.963) (end 113.859351 85.284351) (width 2.2) (layer F.Cu) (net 30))
 (segment (start 113.859351 85.284351) (end 118.202135 85.284351) (width 2.2) (layer F.Cu) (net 30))
 (segment (start 118.202135 85.284351) (end 118.202135 87.503) (width 2.2) (layer F.Cu) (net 30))
 (segment (start 118.202135 87.503) (end 118.202135 89.094351) (width 2.2) (layer F.Cu) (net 30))
 (segment (start 118.202135 89.094351) (end 118.202135 92.904351) (width 2.2) (layer F.Cu) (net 30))
 (segment (start 118.202135 81.474351) (end 118.202135 85.284351) (width 2.2) (layer F.Cu) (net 30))
 (segment (start 177.038 76.15282) (end 177.038 63.5254) (width 0.25) (layer F.Cu) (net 19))
 (segment (start 177.038 63.5254) (end 174.625 61.1124) (width 0.25) (layer F.Cu) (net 19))
 (segment (start 174.625 61.1124) (end 174.625 60.96) (width 0.25) (layer F.Cu) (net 19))
 (segment (start 174.498 77.343) (end 175.84782 77.343) (width 0.25) (layer F.Cu) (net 19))
 (segment (start 175.84782 77.343) (end 177.038 76.15282) (width 0.25) (layer F.Cu) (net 19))
 (segment (start 189.40018 95.123) (end 189.738 95.123) (width 0.25) (layer F.Cu) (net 5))
 (segment (start 189.40018 82.423) (end 189.738 82.423) (width 0.25) (layer F.Cu) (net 10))
 (segment (start 174.83455 84.963) (end 174.498 84.963) (width 0.25) (layer F.Cu) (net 22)))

